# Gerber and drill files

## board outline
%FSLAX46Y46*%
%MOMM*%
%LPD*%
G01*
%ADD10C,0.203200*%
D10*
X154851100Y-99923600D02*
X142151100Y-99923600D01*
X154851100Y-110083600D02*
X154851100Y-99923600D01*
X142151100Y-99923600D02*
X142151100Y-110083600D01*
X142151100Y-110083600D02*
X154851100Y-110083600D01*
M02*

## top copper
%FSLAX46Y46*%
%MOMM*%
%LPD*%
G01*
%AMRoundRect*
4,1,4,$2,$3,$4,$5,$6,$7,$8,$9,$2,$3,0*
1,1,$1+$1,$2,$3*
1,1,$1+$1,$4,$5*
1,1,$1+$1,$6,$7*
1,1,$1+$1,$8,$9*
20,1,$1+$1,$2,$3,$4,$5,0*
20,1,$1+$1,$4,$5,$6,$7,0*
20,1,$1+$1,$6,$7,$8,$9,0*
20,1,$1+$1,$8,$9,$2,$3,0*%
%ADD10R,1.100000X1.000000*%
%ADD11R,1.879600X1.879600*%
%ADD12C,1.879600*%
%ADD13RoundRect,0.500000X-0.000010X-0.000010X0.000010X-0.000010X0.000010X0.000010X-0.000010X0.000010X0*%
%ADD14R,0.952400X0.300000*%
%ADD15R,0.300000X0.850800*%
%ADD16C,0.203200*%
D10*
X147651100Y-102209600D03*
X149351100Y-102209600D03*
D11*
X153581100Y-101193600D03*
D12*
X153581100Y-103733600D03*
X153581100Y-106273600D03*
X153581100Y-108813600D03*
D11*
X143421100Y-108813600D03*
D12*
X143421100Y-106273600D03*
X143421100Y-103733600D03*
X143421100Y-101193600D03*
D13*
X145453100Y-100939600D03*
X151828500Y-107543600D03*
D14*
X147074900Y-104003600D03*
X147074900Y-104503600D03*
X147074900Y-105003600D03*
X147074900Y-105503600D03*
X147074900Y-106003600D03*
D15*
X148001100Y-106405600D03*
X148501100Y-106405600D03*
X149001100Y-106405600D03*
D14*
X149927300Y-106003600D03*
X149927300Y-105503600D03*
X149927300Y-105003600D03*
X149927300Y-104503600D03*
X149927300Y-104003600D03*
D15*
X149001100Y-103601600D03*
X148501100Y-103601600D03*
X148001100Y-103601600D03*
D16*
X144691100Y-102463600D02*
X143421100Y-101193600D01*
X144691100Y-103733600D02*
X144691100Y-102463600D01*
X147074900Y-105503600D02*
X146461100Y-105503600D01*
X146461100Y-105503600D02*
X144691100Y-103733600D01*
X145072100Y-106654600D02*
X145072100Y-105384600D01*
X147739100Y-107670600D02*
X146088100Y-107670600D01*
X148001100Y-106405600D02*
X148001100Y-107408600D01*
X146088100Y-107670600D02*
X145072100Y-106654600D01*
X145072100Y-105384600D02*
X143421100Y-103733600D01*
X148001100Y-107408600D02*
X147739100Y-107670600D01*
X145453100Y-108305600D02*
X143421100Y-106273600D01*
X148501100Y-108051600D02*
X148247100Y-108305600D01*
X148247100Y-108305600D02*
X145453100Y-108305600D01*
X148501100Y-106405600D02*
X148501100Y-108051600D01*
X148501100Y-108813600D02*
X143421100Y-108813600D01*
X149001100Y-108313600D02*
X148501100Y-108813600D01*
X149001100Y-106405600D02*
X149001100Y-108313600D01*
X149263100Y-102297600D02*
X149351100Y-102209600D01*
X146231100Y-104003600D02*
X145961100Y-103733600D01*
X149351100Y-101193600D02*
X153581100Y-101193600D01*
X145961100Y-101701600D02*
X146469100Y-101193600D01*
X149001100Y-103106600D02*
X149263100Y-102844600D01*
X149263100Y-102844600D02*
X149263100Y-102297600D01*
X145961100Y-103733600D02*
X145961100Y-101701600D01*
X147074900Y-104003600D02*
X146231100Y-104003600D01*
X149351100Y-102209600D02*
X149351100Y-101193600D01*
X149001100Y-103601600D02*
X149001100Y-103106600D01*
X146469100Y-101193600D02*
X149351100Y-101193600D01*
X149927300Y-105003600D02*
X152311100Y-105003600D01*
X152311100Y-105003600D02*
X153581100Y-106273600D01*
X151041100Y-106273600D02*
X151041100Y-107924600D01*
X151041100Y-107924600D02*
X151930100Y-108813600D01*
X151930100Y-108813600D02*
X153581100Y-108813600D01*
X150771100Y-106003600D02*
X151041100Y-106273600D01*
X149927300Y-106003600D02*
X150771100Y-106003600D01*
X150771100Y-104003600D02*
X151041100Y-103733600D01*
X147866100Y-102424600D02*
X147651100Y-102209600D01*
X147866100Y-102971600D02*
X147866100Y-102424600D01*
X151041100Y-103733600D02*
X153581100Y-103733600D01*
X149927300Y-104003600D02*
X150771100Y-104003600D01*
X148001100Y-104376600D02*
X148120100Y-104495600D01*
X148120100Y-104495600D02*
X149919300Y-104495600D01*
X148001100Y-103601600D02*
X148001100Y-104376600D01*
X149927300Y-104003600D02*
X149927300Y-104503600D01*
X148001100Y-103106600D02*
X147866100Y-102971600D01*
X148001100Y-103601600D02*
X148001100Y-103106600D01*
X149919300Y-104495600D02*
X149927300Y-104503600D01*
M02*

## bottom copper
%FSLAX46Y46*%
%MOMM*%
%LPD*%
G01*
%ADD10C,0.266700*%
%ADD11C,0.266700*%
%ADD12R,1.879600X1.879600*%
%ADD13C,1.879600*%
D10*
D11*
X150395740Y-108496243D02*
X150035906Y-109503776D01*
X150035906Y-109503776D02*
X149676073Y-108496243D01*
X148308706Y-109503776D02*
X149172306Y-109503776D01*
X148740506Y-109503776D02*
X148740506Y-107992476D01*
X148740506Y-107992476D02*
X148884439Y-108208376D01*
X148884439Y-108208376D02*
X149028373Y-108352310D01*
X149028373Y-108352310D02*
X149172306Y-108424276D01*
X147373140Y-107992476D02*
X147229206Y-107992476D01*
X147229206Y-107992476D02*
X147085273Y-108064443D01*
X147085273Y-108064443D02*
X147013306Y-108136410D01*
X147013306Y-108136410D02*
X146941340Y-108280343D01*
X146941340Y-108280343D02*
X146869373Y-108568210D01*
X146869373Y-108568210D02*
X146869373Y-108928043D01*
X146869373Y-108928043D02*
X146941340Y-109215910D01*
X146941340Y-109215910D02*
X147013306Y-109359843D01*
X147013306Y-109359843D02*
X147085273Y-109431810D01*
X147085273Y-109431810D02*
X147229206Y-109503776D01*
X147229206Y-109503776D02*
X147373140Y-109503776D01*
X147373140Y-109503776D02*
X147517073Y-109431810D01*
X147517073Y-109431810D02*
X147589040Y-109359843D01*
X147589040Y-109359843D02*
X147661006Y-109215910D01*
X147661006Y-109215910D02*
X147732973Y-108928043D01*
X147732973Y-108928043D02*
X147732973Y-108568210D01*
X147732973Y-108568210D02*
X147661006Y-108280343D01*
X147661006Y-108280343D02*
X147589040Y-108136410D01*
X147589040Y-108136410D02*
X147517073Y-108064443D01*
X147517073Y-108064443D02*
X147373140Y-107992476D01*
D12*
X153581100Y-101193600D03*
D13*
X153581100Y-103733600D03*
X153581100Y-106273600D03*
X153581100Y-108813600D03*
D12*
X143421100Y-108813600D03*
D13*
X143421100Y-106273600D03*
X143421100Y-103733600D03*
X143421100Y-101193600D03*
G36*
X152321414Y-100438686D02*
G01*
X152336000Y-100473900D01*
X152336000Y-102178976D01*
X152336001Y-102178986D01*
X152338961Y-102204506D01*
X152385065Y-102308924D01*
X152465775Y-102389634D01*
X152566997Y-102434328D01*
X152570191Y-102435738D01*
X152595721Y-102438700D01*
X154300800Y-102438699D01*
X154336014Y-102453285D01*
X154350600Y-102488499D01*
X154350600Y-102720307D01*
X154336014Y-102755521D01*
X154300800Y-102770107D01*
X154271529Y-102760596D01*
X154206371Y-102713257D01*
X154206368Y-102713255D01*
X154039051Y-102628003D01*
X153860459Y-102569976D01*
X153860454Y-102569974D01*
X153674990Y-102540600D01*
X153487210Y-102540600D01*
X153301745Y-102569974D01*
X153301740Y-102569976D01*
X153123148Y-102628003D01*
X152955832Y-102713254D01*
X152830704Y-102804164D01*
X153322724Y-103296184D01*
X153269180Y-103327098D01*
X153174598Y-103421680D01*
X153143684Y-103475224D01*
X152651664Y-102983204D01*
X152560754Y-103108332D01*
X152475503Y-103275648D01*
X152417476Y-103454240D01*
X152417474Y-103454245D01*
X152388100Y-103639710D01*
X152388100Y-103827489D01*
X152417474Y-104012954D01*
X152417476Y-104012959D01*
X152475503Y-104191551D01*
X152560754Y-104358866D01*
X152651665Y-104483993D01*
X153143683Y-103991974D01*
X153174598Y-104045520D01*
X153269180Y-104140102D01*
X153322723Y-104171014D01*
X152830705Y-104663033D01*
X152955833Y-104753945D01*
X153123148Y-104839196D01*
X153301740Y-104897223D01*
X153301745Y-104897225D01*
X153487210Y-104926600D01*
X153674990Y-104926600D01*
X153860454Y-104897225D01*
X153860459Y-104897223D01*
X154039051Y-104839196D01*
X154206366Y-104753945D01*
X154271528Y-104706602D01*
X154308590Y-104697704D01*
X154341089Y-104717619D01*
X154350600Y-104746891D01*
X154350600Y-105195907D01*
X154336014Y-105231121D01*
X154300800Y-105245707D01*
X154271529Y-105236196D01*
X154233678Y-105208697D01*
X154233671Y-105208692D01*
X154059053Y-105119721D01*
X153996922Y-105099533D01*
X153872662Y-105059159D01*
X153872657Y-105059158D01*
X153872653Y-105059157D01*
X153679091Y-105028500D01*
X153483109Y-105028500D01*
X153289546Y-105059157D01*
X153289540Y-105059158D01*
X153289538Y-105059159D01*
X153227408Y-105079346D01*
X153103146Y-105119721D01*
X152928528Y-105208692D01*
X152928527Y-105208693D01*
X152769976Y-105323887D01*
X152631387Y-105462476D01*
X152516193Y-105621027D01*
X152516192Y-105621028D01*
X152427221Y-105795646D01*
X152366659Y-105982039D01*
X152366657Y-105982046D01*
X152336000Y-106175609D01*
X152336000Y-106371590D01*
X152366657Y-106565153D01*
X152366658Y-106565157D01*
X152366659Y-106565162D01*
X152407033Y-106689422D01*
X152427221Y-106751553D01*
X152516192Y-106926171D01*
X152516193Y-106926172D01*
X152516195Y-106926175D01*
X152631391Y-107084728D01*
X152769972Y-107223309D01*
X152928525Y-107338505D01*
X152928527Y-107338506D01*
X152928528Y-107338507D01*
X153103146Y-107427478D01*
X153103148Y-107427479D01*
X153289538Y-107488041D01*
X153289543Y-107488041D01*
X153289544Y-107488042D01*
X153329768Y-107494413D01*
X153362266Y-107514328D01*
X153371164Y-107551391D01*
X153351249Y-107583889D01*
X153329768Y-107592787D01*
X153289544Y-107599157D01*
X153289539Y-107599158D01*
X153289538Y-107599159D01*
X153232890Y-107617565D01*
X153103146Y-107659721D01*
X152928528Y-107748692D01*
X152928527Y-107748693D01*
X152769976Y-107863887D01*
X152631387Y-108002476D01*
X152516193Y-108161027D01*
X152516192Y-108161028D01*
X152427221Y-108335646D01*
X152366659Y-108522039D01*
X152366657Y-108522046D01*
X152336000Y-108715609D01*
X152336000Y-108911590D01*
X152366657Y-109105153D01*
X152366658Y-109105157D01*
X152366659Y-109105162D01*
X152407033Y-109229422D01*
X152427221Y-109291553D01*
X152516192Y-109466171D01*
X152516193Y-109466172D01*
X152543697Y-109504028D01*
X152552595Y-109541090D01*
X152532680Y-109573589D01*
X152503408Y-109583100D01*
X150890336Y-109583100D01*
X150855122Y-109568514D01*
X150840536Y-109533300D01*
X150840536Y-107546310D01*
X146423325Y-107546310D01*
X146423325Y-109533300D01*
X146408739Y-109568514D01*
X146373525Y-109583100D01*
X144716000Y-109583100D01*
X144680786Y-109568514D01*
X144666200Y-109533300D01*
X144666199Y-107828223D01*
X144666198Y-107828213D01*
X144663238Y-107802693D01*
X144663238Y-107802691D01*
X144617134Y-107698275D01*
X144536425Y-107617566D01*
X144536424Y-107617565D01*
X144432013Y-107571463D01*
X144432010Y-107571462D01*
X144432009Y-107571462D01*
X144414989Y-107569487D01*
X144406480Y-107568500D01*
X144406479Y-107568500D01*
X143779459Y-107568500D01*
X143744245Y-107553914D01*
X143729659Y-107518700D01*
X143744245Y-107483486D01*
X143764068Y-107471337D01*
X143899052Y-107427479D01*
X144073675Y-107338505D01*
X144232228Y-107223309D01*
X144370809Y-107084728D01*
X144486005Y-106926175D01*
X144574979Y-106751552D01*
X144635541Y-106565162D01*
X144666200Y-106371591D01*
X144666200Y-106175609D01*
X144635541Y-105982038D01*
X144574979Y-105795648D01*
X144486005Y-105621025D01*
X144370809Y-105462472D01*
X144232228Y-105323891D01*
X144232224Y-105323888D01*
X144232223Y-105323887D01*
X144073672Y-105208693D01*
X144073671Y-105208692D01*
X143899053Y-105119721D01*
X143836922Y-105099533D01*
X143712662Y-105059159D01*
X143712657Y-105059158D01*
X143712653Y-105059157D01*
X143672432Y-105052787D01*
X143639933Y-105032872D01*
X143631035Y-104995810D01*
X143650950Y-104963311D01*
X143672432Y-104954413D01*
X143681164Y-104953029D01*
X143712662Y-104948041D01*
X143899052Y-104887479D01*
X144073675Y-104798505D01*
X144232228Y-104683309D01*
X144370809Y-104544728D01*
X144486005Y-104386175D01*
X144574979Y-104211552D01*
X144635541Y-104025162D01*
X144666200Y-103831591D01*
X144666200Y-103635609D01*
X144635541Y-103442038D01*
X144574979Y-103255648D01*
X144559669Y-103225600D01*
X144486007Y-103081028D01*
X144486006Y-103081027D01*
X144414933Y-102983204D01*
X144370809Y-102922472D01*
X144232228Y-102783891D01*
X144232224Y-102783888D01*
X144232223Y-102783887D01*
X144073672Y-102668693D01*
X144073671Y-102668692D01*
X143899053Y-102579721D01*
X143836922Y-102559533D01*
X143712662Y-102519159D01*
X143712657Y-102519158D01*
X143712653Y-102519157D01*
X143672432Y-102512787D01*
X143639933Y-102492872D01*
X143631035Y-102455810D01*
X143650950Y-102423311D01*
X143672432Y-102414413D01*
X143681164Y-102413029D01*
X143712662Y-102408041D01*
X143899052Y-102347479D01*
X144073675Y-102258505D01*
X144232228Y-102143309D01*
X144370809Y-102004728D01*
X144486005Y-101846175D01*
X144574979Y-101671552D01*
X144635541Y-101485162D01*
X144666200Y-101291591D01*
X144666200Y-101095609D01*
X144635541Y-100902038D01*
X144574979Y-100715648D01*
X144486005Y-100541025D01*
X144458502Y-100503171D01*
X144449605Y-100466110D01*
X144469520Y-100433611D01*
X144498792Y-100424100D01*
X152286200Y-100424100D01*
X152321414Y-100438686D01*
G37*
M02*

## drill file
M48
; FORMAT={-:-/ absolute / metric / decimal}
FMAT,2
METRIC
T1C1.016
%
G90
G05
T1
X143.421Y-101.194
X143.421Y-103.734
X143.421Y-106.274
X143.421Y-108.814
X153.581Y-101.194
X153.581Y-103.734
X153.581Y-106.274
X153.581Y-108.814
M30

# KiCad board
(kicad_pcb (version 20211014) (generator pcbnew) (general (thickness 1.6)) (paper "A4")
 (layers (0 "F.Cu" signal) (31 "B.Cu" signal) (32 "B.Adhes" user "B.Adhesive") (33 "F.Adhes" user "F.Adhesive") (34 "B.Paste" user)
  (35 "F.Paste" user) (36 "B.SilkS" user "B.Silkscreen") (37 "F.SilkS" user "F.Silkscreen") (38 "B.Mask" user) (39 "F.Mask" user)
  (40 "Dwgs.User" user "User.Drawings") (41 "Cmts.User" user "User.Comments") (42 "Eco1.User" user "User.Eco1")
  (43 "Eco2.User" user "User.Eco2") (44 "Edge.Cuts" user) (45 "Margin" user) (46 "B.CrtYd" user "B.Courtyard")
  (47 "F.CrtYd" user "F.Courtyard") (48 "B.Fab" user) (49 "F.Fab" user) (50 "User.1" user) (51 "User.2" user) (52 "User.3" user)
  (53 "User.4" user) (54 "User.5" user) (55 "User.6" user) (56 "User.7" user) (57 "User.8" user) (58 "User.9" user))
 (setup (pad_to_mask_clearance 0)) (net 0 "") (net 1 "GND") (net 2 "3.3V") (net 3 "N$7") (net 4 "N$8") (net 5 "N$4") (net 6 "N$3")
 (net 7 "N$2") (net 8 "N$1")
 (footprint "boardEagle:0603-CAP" (layer "F.Cu") (at 148.5011 102.2096)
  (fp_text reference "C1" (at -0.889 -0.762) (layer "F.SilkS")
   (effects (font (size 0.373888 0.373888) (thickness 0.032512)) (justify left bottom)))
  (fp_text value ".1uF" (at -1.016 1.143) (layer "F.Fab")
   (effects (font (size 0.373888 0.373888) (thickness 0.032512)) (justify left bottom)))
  (pad "1" smd rect (at -0.85 0) (size 1.1 1) (layers "F.Cu" "F.Paste" "F.Mask") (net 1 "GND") (solder_mask_margin 0.1016))
  (pad "2" smd rect (at 0.85 0) (size 1.1 1) (layers "F.Cu" "F.Paste" "F.Mask") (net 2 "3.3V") (solder_mask_margin 0.1016)))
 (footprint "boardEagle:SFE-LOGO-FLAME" (layer "F.Cu") (at 145.9611 109.7026)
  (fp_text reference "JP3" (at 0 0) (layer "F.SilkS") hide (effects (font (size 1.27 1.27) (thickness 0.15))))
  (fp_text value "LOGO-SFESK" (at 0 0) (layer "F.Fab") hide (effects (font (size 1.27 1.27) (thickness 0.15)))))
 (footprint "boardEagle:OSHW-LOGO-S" (layer "F.Cu") (at 150.0251 108.5596)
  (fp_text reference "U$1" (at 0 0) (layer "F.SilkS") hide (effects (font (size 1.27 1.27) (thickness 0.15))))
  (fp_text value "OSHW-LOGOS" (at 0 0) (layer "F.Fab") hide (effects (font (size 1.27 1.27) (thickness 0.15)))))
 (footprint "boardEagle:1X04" (layer "F.Cu") (at 153.5811 101.1936 -90)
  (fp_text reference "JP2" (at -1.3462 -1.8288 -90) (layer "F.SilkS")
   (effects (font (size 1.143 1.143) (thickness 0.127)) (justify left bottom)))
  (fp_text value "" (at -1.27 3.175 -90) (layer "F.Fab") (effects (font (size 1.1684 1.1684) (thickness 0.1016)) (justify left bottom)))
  (pad "1" thru_hole rect (at 0 0) (size 1.8796 1.8796) (drill 1.016) (layers *.Cu *.Mask) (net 2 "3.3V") (solder_mask_margin 0.1016))
  (pad "2" thru_hole circle (at 2.54 0) (size 1.8796 1.8796) (drill 1.016) (layers *.Cu *.Mask) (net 1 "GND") (solder_mask_margin 0.1016))
  (pad "3" thru_hole circle (at 5.08 0) (size 1.8796 1.8796) (drill 1.016) (layers *.Cu *.Mask) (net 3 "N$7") (solder_mask_margin 0.1016))
  (pad "4" thru_hole circle (at 7.62 0) (size 1.8796 1.8796) (drill 1.016) (layers *.Cu *.Mask) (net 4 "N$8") (solder_mask_margin 0.1016)))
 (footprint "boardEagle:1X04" (layer "F.Cu") (at 143.4211 108.8136 90)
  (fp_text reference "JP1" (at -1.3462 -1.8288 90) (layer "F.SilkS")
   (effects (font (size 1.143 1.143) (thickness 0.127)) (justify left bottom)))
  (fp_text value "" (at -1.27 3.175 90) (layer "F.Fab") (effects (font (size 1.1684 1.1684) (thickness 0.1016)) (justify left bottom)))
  (pad "1" thru_hole rect (at 0 0 180) (size 1.8796 1.8796) (drill 1.016) (layers *.Cu *.Mask) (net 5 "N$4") (solder_mask_margin 0.1016))
  (pad "2" thru_hole circle (at 2.54 0 180) (size 1.8796 1.8796) (drill 1.016) (layers *.Cu *.Mask) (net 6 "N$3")
   (solder_mask_margin 0.1016))
  (pad "3" thru_hole circle (at 5.08 0 180) (size 1.8796 1.8796) (drill 1.016) (layers *.Cu *.Mask) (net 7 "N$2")
   (solder_mask_margin 0.1016))
  (pad "4" thru_hole circle (at 7.62 0 180) (size 1.8796 1.8796) (drill 1.016) (layers *.Cu *.Mask) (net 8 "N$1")
   (solder_mask_margin 0.1016)))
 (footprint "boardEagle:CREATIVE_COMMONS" (layer "F.Cu") (at 64.6811 108.8136)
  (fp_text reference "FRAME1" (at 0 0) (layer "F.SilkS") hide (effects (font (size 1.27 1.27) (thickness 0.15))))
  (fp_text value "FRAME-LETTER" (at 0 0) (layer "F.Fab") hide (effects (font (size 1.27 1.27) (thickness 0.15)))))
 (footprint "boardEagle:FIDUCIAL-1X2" (layer "F.Cu") (at 145.4531 100.9396)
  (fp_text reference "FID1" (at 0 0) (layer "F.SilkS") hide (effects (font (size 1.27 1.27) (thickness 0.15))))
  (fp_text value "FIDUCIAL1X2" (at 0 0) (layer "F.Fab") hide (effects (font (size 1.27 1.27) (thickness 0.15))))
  (pad "1" smd roundrect (at 0 0) (size 1 1) (layers "F.Cu" "F.Mask") (roundrect_rratio 0.5) (solder_mask_margin 0.1016)))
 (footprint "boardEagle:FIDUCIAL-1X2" (layer "F.Cu") (at 151.8285 107.5436)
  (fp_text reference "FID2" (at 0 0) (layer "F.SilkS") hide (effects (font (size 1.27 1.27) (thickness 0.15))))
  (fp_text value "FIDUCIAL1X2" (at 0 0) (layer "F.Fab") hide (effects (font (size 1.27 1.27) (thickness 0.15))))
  (pad "1" smd roundrect (at 0 0) (size 1 1) (layers "F.Cu" "F.Mask") (roundrect_rratio 0.5) (solder_mask_margin 0.1016)))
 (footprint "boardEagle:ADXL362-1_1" (layer "F.Cu") (at 148.5011 105.0036)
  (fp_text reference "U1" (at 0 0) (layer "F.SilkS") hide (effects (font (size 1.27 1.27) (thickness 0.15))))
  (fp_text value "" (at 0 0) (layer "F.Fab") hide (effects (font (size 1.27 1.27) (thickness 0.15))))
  (pad "P$1" smd rect (at -1.4262 -1) (size 0.9524 0.3) (layers "F.Cu" "F.Paste" "F.Mask") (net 2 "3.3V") (solder_mask_margin 0.1016))
  (pad "P$2" smd rect (at -1.4262 -0.5) (size 0.9524 0.3) (layers "F.Cu" "F.Paste" "F.Mask") (solder_mask_margin 0.1016))
  (pad "P$3" smd rect (at -1.4262 0) (size 0.9524 0.3) (layers "F.Cu" "F.Paste" "F.Mask") (solder_mask_margin 0.1016))
  (pad "P$4" smd rect (at -1.4262 0.5) (size 0.9524 0.3) (layers "F.Cu" "F.Paste" "F.Mask") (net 8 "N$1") (solder_mask_margin 0.1016))
  (pad "P$5" smd rect (at -1.4262 1) (size 0.9524 0.3) (layers "F.Cu" "F.Paste" "F.Mask") (solder_mask_margin 0.1016))
  (pad "P$6" smd rect (at -0.5 1.402 90) (size 0.8508 0.3) (layers "F.Cu" "F.Paste" "F.Mask") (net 7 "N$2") (solder_mask_margin 0.1016))
  (pad "P$7" smd rect (at 0 1.402 90) (size 0.8508 0.3) (layers "F.Cu" "F.Paste" "F.Mask") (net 6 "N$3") (solder_mask_margin 0.1016))
  (pad "P$8" smd rect (at 0.5 1.402 90) (size 0.8508 0.3) (layers "F.Cu" "F.Paste" "F.Mask") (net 5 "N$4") (solder_mask_margin 0.1016))
  (pad "P$9" smd rect (at 1.4262 1) (size 0.9524 0.3) (layers "F.Cu" "F.Paste" "F.Mask") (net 4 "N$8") (solder_mask_margin 0.1016))
  (pad "P$10" smd rect (at 1.4262 0.5) (size 0.9524 0.3) (layers "F.Cu" "F.Paste" "F.Mask") (solder_mask_margin 0.1016))
  (pad "P$11" smd rect (at 1.4262 0) (size 0.9524 0.3) (layers "F.Cu" "F.Paste" "F.Mask") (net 3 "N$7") (solder_mask_margin 0.1016))
  (pad "P$12" smd rect (at 1.4262 -0.5) (size 0.9524 0.3) (layers "F.Cu" "F.Paste" "F.Mask") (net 1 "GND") (solder_mask_margin 0.1016))
  (pad "P$13" smd rect (at 1.4262 -1) (size 0.9524 0.3) (layers "F.Cu" "F.Paste" "F.Mask") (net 1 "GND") (solder_mask_margin 0.1016))
  (pad "P$14" smd rect (at 0.5 -1.402 90) (size 0.8508 0.3) (layers "F.Cu" "F.Paste" "F.Mask") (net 2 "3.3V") (solder_mask_margin 0.1016))
  (pad "P$15" smd rect (at 0 -1.402 90) (size 0.8508 0.3) (layers "F.Cu" "F.Paste" "F.Mask") (solder_mask_margin 0.1016))
  (pad "P$16" smd rect (at -0.5 -1.402 90) (size 0.8508 0.3) (layers "F.Cu" "F.Paste" "F.Mask") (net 1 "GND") (solder_mask_margin 0.1016)))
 (gr_line (start 154.8511 99.9236) (end 142.1511 99.9236) (layer "Edge.Cuts") (width 0.2032))
 (gr_line (start 154.8511 110.0836) (end 154.8511 99.9236) (layer "Edge.Cuts") (width 0.2032))
 (gr_line (start 142.1511 99.9236) (end 142.1511 110.0836) (layer "Edge.Cuts") (width 0.2032))
 (gr_line (start 142.1511 110.0836) (end 154.8511 110.0836) (layer "Edge.Cuts") (width 0.2032))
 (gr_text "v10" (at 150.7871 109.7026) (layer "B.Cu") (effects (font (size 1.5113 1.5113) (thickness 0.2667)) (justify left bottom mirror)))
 (segment (start 144.6911 102.4636) (end 143.4211 101.1936) (width 0.2032) (layer "F.Cu") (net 8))
 (segment (start 144.6911 103.7336) (end 144.6911 102.4636) (width 0.2032) (layer "F.Cu") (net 8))
 (segment (start 147.0749 105.5036) (end 146.4611 105.5036) (width 0.2032) (layer "F.Cu") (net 8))
 (segment (start 146.4611 105.5036) (end 144.6911 103.7336) (width 0.2032) (layer "F.Cu") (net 8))
 (segment (start 145.0721 106.6546) (end 145.0721 105.3846) (width 0.2032) (layer "F.Cu") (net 7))
 (segment (start 147.7391 107.6706) (end 146.0881 107.6706) (width 0.2032) (layer "F.Cu") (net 7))
 (segment (start 148.0011 106.4056) (end 148.0011 107.4086) (width 0.2032) (layer "F.Cu") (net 7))
 (segment (start 146.0881 107.6706) (end 145.0721 106.6546) (width 0.2032) (layer "F.Cu") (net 7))
 (segment (start 145.0721 105.3846) (end 143.4211 103.7336) (width 0.2032) (layer "F.Cu") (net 7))
 (segment (start 148.0011 107.4086) (end 147.7391 107.6706) (width 0.2032) (layer "F.Cu") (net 7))
 (segment (start 145.4531 108.3056) (end 143.4211 106.2736) (width 0.2032) (layer "F.Cu") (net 6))
 (segment (start 148.5011 108.0516) (end 148.2471 108.3056) (width 0.2032) (layer "F.Cu") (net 6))
 (segment (start 148.2471 108.3056) (end 145.4531 108.3056) (width 0.2032) (layer "F.Cu") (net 6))
 (segment (start 148.5011 106.4056) (end 148.5011 108.0516) (width 0.2032) (layer "F.Cu") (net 6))
 (segment (start 148.5011 108.8136) (end 143.4211 108.8136) (width 0.2032) (layer "F.Cu") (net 5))
 (segment (start 149.0011 108.3136) (end 148.5011 108.8136) (width 0.2032) (layer "F.Cu") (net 5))
 (segment (start 149.0011 106.4056) (end 149.0011 108.3136) (width 0.2032) (layer "F.Cu") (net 5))
 (segment (start 149.2631 102.2976) (end 149.3511 102.2096) (width 0.2032) (layer "F.Cu") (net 2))
 (segment (start 146.2311 104.0036) (end 145.9611 103.7336) (width 0.2032) (layer "F.Cu") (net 2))
 (segment (start 149.3511 101.1936) (end 153.5811 101.1936) (width 0.2032) (layer "F.Cu") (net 2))
 (segment (start 145.9611 101.7016) (end 146.4691 101.1936) (width 0.2032) (layer "F.Cu") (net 2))
 (segment (start 149.0011 103.1066) (end 149.2631 102.8446) (width 0.2032) (layer "F.Cu") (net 2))
 (segment (start 149.2631 102.8446) (end 149.2631 102.2976) (width 0.2032) (layer "F.Cu") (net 2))
 (segment (start 145.9611 103.7336) (end 145.9611 101.7016) (width 0.2032) (layer "F.Cu") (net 2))
 (segment (start 147.0749 104.0036) (end 146.2311 104.0036) (width 0.2032) (layer "F.Cu") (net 2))
 (segment (start 149.3511 102.2096) (end 149.3511 101.1936) (width 0.2032) (layer "F.Cu") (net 2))
 (segment (start 149.0011 103.6016) (end 149.0011 103.1066) (width 0.2032) (layer "F.Cu") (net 2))
 (segment (start 146.4691 101.1936) (end 149.3511 101.1936) (width 0.2032) (layer "F.Cu") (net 2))
 (segment (start 149.9273 105.0036) (end 152.3111 105.0036) (width 0.2032) (layer "F.Cu") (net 3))
 (segment (start 152.3111 105.0036) (end 153.5811 106.2736) (width 0.2032) (layer "F.Cu") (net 3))
 (segment (start 151.0411 106.2736) (end 151.0411 107.9246) (width 0.2032) (layer "F.Cu") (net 4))
 (segment (start 151.0411 107.9246) (end 151.9301 108.8136) (width 0.2032) (layer "F.Cu") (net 4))
 (segment (start 151.9301 108.8136) (end 153.5811 108.8136) (width 0.2032) (layer "F.Cu") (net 4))
 (segment (start 150.7711 106.0036) (end 151.0411 106.2736) (width 0.2032) (layer "F.Cu") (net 4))
 (segment (start 149.9273 106.0036) (end 150.7711 106.0036) (width 0.2032) (layer "F.Cu") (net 4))
 (segment (start 150.7711 104.0036) (end 151.0411 103.7336) (width 0.2032) (layer "F.Cu") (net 1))
 (segment (start 147.8661 102.4246) (end 147.6511 102.2096) (width 0.2032) (layer "F.Cu") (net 1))
 (segment (start 147.8661 102.9716) (end 147.8661 102.4246) (width 0.2032) (layer "F.Cu") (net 1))
 (segment (start 151.0411 103.7336) (end 153.5811 103.7336) (width 0.2032) (layer "F.Cu") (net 1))
 (segment (start 149.9273 104.0036) (end 150.7711 104.0036) (width 0.2032) (layer "F.Cu") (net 1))
 (segment (start 148.0011 104.3766) (end 148.1201 104.4956) (width 0.2032) (layer "F.Cu") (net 1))
 (segment (start 148.1201 104.4956) (end 149.9193 104.4956) (width 0.2032) (layer "F.Cu") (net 1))
 (segment (start 148.0011 103.6016) (end 148.0011 104.3766) (width 0.2032) (layer "F.Cu") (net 1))
 (segment (start 149.9273 104.0036) (end 149.9273 104.5036) (width 0.2032) (layer "F.Cu") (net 1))
 (segment (start 148.0011 103.1066) (end 147.8661 102.9716) (width 0.2032) (layer "F.Cu") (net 1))
 (segment (start 148.0011 103.6016) (end 148.0011 103.1066) (width 0.2032) (layer "F.Cu") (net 1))
 (segment (start 149.9193 104.4956) (end 149.9273 104.5036) (width 0.2032) (layer "F.Cu") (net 1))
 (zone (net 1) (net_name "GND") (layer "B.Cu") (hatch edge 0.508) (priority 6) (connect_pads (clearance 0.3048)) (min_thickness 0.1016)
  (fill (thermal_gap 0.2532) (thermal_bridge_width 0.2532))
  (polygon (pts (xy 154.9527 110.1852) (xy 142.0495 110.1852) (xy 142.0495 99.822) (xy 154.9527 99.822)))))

